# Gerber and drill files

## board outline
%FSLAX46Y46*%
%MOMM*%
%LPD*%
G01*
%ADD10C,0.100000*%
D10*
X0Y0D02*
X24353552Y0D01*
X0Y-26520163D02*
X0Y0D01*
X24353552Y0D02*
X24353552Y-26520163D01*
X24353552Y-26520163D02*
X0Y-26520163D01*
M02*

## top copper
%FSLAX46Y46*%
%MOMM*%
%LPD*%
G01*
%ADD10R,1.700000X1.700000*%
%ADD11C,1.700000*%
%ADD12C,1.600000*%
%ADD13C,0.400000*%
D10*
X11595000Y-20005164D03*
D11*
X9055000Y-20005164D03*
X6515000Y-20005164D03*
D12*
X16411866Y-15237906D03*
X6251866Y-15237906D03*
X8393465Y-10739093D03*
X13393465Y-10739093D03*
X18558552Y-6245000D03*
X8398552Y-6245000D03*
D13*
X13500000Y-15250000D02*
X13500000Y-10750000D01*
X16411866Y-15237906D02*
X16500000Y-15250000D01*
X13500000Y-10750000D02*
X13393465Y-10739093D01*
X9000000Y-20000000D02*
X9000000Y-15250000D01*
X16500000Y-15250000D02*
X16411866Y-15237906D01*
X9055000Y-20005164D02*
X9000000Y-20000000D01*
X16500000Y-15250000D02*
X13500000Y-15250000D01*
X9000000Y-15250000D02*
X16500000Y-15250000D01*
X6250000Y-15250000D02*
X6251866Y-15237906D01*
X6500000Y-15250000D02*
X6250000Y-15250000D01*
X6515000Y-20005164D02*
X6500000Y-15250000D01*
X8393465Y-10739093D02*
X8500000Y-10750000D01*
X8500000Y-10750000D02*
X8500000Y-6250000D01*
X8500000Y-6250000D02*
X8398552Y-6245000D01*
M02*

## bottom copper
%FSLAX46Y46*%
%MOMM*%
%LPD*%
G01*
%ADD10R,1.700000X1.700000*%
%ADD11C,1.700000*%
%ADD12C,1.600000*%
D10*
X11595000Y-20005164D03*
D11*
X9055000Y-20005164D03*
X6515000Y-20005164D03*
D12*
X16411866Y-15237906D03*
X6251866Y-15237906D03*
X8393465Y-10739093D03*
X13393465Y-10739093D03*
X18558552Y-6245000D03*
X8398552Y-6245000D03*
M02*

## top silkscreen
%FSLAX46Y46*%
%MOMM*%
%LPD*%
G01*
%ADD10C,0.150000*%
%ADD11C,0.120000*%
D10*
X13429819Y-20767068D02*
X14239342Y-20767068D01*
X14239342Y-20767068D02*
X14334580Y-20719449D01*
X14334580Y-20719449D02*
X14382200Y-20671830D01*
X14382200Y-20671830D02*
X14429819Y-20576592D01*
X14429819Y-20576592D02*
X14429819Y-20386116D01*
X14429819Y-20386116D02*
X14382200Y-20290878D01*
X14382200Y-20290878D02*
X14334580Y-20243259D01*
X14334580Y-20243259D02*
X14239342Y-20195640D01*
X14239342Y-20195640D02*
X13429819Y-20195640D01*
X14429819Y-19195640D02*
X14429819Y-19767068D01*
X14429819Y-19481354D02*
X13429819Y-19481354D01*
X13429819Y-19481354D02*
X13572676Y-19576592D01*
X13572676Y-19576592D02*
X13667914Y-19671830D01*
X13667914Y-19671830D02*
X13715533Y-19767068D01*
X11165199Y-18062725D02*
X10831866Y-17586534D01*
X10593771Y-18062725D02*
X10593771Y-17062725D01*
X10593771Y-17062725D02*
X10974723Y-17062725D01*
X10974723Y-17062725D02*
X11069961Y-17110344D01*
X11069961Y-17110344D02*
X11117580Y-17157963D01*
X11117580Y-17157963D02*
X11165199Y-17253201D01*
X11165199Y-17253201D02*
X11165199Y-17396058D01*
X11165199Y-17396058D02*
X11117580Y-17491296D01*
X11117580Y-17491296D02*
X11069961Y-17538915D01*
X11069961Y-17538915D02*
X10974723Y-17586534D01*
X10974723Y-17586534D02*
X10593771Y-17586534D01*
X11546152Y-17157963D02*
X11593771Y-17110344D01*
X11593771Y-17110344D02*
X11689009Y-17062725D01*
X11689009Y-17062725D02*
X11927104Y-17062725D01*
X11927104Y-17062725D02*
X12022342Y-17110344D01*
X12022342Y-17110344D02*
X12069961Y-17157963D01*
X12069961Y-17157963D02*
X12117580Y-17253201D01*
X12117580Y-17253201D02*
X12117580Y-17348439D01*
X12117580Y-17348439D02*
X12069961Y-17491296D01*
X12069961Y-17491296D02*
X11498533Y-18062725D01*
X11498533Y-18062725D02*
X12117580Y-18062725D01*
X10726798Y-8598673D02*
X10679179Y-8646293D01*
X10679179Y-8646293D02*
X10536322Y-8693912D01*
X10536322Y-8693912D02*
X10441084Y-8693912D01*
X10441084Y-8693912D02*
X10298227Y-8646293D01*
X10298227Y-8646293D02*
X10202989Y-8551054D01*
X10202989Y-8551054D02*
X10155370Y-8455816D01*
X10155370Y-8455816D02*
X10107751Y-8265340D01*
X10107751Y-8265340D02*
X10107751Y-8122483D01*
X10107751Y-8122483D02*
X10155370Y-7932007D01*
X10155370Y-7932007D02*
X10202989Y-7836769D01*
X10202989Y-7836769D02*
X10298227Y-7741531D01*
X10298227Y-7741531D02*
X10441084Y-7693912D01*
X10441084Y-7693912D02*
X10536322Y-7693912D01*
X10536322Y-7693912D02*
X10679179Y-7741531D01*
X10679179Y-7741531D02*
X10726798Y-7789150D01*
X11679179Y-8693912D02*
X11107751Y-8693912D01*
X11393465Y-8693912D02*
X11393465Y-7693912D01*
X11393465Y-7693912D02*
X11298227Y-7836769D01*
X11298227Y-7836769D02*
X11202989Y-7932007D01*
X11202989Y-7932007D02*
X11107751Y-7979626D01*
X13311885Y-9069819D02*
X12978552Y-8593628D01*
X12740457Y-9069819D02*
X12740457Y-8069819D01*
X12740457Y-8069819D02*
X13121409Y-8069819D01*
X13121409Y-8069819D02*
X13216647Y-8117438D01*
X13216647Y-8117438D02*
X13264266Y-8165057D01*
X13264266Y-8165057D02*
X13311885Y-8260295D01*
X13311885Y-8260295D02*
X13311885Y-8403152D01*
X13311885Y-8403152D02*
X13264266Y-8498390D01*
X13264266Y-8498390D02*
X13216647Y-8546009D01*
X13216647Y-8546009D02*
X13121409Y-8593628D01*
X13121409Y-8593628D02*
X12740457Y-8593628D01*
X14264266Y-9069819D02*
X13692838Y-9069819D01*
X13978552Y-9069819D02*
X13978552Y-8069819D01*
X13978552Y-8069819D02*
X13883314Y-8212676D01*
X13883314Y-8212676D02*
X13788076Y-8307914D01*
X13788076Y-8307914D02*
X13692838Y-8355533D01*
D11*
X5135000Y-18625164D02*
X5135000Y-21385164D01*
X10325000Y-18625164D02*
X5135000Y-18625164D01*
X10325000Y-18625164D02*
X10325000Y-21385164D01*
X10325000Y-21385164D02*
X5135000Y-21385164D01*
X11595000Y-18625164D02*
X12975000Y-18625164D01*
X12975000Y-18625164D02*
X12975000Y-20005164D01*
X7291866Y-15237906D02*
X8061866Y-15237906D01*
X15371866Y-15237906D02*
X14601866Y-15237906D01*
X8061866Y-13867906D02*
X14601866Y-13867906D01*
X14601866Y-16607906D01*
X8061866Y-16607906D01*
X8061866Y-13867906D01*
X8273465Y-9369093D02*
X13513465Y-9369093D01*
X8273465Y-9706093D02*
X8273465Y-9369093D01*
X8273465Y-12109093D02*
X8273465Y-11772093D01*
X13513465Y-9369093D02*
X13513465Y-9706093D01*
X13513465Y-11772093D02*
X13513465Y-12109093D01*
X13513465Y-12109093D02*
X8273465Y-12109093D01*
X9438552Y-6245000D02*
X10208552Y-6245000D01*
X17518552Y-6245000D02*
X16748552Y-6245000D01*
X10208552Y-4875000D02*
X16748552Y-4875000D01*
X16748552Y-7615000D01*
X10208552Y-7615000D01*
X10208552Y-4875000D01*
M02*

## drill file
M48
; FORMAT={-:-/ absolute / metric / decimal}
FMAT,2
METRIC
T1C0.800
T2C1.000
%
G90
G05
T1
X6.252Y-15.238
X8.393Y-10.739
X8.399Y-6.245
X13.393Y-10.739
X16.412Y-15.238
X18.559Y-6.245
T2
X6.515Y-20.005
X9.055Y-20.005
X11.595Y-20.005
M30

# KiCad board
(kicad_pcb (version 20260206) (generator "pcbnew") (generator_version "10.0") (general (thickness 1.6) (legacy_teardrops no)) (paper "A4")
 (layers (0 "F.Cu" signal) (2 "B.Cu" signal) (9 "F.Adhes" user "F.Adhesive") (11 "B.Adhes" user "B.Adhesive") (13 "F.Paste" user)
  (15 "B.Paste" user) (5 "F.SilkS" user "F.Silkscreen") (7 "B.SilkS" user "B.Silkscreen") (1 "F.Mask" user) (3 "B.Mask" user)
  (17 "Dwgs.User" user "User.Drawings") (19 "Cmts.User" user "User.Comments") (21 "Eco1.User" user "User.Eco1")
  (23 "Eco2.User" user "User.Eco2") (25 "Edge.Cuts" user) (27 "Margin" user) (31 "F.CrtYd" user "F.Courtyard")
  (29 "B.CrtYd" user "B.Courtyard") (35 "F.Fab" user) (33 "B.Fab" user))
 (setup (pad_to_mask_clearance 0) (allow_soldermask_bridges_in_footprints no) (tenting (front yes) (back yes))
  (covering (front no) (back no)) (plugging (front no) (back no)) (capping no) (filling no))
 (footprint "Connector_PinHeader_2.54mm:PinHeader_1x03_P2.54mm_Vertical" (layer "F.Cu") (at 11.595 20.005164 -90)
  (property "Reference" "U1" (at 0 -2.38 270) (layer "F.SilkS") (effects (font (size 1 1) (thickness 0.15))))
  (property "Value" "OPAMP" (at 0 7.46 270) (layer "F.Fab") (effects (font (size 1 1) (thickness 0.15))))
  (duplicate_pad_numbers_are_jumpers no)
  (fp_line (start -1.38 6.46) (end 1.38 6.46) (stroke (width 0.12) (type solid)) (layer "F.SilkS"))
  (fp_line (start -1.38 1.27) (end -1.38 6.46) (stroke (width 0.12) (type solid)) (layer "F.SilkS"))
  (fp_line (start -1.38 1.27) (end 1.38 1.27) (stroke (width 0.12) (type solid)) (layer "F.SilkS"))
  (fp_line (start 1.38 1.27) (end 1.38 6.46) (stroke (width 0.12) (type solid)) (layer "F.SilkS"))
  (fp_line (start -1.38 0) (end -1.38 -1.38) (stroke (width 0.12) (type solid)) (layer "F.SilkS"))
  (fp_line (start -1.38 -1.38) (end 0 -1.38) (stroke (width 0.12) (type solid)) (layer "F.SilkS"))
  (pad "1" thru_hole rect (at 0 0 270) (size 1.7 1.7) (drill 1) (layers "*.Cu" "*.Mask") (remove_unused_layers no))
  (pad "2" thru_hole circle (at 0 2.54 270) (size 1.7 1.7) (drill 1) (layers "*.Cu" "*.Mask") (remove_unused_layers no) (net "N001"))
  (pad "3" thru_hole circle (at 0 5.08 270) (size 1.7 1.7) (drill 1) (layers "*.Cu" "*.Mask") (remove_unused_layers no) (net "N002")))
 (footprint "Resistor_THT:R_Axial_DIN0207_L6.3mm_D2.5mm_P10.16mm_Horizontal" (layer "F.Cu") (at 16.411866 15.237906 180)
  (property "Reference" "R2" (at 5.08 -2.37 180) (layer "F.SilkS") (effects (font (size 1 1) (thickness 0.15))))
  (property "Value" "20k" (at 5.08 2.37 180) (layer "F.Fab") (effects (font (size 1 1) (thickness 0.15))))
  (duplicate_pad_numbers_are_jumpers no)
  (fp_line (start 9.12 0) (end 8.35 0) (stroke (width 0.12) (type solid)) (layer "F.SilkS"))
  (fp_line (start 1.04 0) (end 1.81 0) (stroke (width 0.12) (type solid)) (layer "F.SilkS"))
  (fp_rect (start 1.81 -1.37) (end 8.35 1.37) (stroke (width 0.12) (type solid)) (fill no) (layer "F.SilkS"))
  (pad "1" thru_hole circle (at 0 0 180) (size 1.6 1.6) (drill 0.8) (layers "*.Cu" "*.Mask") (remove_unused_layers no) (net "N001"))
  (pad "2" thru_hole circle (at 10.16 0 180) (size 1.6 1.6) (drill 0.8) (layers "*.Cu" "*.Mask") (remove_unused_layers no) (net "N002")))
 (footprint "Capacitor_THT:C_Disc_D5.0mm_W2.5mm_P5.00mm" (layer "F.Cu") (at 8.393465 10.739093)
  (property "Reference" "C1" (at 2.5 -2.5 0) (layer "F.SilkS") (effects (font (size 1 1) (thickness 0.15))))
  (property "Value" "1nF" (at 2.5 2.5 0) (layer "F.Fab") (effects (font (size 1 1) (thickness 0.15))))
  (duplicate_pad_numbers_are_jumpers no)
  (fp_line (start -0.12 -1.37) (end 5.12 -1.37) (stroke (width 0.12) (type solid)) (layer "F.SilkS"))
  (fp_line (start -0.12 -1.033) (end -0.12 -1.37) (stroke (width 0.12) (type solid)) (layer "F.SilkS"))
  (fp_line (start -0.12 1.37) (end -0.12 1.033) (stroke (width 0.12) (type solid)) (layer "F.SilkS"))
  (fp_line (start 5.12 -1.37) (end 5.12 -1.033) (stroke (width 0.12) (type solid)) (layer "F.SilkS"))
  (fp_line (start 5.12 1.033) (end 5.12 1.37) (stroke (width 0.12) (type solid)) (layer "F.SilkS"))
  (fp_line (start 5.12 1.37) (end -0.12 1.37) (stroke (width 0.12) (type solid)) (layer "F.SilkS"))
  (pad "1" thru_hole circle (at 0 0) (size 1.6 1.6) (drill 0.8) (layers "*.Cu" "*.Mask") (remove_unused_layers no) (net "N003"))
  (pad "2" thru_hole circle (at 5 0) (size 1.6 1.6) (drill 0.8) (layers "*.Cu" "*.Mask") (remove_unused_layers no) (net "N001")))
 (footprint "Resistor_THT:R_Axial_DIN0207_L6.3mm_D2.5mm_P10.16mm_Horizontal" (layer "F.Cu") (at 18.558552 6.245 180)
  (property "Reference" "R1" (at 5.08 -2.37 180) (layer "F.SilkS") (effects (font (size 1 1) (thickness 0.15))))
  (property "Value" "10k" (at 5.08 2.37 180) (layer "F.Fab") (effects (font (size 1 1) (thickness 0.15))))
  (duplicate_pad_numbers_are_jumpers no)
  (fp_line (start 9.12 0) (end 8.35 0) (stroke (width 0.12) (type solid)) (layer "F.SilkS"))
  (fp_line (start 1.04 0) (end 1.81 0) (stroke (width 0.12) (type solid)) (layer "F.SilkS"))
  (fp_rect (start 1.81 -1.37) (end 8.35 1.37) (stroke (width 0.12) (type solid)) (fill no) (layer "F.SilkS"))
  (pad "1" thru_hole circle (at 0 0 180) (size 1.6 1.6) (drill 0.8) (layers "*.Cu" "*.Mask") (remove_unused_layers no))
  (pad "2" thru_hole circle (at 10.16 0 180) (size 1.6 1.6) (drill 0.8) (layers "*.Cu" "*.Mask") (remove_unused_layers no) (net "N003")))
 (gr_line (start 0 0) (end 24.353552 0) (stroke (width 0.1) (type default)) (layer "Edge.Cuts"))
 (gr_line (start 0 26.520163) (end 0 0) (stroke (width 0.1) (type default)) (layer "Edge.Cuts"))
 (gr_line (start 24.353552 0) (end 24.353552 26.520163) (stroke (width 0.1) (type default)) (layer "Edge.Cuts"))
 (gr_line (start 24.353552 26.520163) (end 0 26.520163) (stroke (width 0.1) (type default)) (layer "Edge.Cuts"))
 (segment (start 13.5 15.25) (end 13.5 10.75) (width 0.4) (layer "F.Cu") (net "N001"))
 (segment (start 16.411866 15.237906) (end 16.5 15.25) (width 0.4) (layer "F.Cu") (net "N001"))
 (segment (start 13.5 10.75) (end 13.393465 10.739093) (width 0.4) (layer "F.Cu") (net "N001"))
 (segment (start 9 20) (end 9 15.25) (width 0.4) (layer "F.Cu") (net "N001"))
 (segment (start 16.5 15.25) (end 16.411866 15.237906) (width 0.4) (layer "F.Cu") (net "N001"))
 (segment (start 9.055 20.005164) (end 9 20) (width 0.4) (layer "F.Cu") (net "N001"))
 (segment (start 16.5 15.25) (end 13.5 15.25) (width 0.4) (layer "F.Cu") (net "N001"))
 (segment (start 9 15.25) (end 16.5 15.25) (width 0.4) (layer "F.Cu") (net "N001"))
 (segment (start 6.25 15.25) (end 6.251866 15.237906) (width 0.4) (layer "F.Cu") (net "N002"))
 (segment (start 6.5 15.25) (end 6.25 15.25) (width 0.4) (layer "F.Cu") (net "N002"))
 (segment (start 6.515 20.005164) (end 6.5 15.25) (width 0.4) (layer "F.Cu") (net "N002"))
 (segment (start 8.393465 10.739093) (end 8.5 10.75) (width 0.4) (layer "F.Cu") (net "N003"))
 (segment (start 8.5 10.75) (end 8.5 6.25) (width 0.4) (layer "F.Cu") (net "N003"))
 (segment (start 8.5 6.25) (end 8.398552 6.245) (width 0.4) (layer "F.Cu") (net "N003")))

